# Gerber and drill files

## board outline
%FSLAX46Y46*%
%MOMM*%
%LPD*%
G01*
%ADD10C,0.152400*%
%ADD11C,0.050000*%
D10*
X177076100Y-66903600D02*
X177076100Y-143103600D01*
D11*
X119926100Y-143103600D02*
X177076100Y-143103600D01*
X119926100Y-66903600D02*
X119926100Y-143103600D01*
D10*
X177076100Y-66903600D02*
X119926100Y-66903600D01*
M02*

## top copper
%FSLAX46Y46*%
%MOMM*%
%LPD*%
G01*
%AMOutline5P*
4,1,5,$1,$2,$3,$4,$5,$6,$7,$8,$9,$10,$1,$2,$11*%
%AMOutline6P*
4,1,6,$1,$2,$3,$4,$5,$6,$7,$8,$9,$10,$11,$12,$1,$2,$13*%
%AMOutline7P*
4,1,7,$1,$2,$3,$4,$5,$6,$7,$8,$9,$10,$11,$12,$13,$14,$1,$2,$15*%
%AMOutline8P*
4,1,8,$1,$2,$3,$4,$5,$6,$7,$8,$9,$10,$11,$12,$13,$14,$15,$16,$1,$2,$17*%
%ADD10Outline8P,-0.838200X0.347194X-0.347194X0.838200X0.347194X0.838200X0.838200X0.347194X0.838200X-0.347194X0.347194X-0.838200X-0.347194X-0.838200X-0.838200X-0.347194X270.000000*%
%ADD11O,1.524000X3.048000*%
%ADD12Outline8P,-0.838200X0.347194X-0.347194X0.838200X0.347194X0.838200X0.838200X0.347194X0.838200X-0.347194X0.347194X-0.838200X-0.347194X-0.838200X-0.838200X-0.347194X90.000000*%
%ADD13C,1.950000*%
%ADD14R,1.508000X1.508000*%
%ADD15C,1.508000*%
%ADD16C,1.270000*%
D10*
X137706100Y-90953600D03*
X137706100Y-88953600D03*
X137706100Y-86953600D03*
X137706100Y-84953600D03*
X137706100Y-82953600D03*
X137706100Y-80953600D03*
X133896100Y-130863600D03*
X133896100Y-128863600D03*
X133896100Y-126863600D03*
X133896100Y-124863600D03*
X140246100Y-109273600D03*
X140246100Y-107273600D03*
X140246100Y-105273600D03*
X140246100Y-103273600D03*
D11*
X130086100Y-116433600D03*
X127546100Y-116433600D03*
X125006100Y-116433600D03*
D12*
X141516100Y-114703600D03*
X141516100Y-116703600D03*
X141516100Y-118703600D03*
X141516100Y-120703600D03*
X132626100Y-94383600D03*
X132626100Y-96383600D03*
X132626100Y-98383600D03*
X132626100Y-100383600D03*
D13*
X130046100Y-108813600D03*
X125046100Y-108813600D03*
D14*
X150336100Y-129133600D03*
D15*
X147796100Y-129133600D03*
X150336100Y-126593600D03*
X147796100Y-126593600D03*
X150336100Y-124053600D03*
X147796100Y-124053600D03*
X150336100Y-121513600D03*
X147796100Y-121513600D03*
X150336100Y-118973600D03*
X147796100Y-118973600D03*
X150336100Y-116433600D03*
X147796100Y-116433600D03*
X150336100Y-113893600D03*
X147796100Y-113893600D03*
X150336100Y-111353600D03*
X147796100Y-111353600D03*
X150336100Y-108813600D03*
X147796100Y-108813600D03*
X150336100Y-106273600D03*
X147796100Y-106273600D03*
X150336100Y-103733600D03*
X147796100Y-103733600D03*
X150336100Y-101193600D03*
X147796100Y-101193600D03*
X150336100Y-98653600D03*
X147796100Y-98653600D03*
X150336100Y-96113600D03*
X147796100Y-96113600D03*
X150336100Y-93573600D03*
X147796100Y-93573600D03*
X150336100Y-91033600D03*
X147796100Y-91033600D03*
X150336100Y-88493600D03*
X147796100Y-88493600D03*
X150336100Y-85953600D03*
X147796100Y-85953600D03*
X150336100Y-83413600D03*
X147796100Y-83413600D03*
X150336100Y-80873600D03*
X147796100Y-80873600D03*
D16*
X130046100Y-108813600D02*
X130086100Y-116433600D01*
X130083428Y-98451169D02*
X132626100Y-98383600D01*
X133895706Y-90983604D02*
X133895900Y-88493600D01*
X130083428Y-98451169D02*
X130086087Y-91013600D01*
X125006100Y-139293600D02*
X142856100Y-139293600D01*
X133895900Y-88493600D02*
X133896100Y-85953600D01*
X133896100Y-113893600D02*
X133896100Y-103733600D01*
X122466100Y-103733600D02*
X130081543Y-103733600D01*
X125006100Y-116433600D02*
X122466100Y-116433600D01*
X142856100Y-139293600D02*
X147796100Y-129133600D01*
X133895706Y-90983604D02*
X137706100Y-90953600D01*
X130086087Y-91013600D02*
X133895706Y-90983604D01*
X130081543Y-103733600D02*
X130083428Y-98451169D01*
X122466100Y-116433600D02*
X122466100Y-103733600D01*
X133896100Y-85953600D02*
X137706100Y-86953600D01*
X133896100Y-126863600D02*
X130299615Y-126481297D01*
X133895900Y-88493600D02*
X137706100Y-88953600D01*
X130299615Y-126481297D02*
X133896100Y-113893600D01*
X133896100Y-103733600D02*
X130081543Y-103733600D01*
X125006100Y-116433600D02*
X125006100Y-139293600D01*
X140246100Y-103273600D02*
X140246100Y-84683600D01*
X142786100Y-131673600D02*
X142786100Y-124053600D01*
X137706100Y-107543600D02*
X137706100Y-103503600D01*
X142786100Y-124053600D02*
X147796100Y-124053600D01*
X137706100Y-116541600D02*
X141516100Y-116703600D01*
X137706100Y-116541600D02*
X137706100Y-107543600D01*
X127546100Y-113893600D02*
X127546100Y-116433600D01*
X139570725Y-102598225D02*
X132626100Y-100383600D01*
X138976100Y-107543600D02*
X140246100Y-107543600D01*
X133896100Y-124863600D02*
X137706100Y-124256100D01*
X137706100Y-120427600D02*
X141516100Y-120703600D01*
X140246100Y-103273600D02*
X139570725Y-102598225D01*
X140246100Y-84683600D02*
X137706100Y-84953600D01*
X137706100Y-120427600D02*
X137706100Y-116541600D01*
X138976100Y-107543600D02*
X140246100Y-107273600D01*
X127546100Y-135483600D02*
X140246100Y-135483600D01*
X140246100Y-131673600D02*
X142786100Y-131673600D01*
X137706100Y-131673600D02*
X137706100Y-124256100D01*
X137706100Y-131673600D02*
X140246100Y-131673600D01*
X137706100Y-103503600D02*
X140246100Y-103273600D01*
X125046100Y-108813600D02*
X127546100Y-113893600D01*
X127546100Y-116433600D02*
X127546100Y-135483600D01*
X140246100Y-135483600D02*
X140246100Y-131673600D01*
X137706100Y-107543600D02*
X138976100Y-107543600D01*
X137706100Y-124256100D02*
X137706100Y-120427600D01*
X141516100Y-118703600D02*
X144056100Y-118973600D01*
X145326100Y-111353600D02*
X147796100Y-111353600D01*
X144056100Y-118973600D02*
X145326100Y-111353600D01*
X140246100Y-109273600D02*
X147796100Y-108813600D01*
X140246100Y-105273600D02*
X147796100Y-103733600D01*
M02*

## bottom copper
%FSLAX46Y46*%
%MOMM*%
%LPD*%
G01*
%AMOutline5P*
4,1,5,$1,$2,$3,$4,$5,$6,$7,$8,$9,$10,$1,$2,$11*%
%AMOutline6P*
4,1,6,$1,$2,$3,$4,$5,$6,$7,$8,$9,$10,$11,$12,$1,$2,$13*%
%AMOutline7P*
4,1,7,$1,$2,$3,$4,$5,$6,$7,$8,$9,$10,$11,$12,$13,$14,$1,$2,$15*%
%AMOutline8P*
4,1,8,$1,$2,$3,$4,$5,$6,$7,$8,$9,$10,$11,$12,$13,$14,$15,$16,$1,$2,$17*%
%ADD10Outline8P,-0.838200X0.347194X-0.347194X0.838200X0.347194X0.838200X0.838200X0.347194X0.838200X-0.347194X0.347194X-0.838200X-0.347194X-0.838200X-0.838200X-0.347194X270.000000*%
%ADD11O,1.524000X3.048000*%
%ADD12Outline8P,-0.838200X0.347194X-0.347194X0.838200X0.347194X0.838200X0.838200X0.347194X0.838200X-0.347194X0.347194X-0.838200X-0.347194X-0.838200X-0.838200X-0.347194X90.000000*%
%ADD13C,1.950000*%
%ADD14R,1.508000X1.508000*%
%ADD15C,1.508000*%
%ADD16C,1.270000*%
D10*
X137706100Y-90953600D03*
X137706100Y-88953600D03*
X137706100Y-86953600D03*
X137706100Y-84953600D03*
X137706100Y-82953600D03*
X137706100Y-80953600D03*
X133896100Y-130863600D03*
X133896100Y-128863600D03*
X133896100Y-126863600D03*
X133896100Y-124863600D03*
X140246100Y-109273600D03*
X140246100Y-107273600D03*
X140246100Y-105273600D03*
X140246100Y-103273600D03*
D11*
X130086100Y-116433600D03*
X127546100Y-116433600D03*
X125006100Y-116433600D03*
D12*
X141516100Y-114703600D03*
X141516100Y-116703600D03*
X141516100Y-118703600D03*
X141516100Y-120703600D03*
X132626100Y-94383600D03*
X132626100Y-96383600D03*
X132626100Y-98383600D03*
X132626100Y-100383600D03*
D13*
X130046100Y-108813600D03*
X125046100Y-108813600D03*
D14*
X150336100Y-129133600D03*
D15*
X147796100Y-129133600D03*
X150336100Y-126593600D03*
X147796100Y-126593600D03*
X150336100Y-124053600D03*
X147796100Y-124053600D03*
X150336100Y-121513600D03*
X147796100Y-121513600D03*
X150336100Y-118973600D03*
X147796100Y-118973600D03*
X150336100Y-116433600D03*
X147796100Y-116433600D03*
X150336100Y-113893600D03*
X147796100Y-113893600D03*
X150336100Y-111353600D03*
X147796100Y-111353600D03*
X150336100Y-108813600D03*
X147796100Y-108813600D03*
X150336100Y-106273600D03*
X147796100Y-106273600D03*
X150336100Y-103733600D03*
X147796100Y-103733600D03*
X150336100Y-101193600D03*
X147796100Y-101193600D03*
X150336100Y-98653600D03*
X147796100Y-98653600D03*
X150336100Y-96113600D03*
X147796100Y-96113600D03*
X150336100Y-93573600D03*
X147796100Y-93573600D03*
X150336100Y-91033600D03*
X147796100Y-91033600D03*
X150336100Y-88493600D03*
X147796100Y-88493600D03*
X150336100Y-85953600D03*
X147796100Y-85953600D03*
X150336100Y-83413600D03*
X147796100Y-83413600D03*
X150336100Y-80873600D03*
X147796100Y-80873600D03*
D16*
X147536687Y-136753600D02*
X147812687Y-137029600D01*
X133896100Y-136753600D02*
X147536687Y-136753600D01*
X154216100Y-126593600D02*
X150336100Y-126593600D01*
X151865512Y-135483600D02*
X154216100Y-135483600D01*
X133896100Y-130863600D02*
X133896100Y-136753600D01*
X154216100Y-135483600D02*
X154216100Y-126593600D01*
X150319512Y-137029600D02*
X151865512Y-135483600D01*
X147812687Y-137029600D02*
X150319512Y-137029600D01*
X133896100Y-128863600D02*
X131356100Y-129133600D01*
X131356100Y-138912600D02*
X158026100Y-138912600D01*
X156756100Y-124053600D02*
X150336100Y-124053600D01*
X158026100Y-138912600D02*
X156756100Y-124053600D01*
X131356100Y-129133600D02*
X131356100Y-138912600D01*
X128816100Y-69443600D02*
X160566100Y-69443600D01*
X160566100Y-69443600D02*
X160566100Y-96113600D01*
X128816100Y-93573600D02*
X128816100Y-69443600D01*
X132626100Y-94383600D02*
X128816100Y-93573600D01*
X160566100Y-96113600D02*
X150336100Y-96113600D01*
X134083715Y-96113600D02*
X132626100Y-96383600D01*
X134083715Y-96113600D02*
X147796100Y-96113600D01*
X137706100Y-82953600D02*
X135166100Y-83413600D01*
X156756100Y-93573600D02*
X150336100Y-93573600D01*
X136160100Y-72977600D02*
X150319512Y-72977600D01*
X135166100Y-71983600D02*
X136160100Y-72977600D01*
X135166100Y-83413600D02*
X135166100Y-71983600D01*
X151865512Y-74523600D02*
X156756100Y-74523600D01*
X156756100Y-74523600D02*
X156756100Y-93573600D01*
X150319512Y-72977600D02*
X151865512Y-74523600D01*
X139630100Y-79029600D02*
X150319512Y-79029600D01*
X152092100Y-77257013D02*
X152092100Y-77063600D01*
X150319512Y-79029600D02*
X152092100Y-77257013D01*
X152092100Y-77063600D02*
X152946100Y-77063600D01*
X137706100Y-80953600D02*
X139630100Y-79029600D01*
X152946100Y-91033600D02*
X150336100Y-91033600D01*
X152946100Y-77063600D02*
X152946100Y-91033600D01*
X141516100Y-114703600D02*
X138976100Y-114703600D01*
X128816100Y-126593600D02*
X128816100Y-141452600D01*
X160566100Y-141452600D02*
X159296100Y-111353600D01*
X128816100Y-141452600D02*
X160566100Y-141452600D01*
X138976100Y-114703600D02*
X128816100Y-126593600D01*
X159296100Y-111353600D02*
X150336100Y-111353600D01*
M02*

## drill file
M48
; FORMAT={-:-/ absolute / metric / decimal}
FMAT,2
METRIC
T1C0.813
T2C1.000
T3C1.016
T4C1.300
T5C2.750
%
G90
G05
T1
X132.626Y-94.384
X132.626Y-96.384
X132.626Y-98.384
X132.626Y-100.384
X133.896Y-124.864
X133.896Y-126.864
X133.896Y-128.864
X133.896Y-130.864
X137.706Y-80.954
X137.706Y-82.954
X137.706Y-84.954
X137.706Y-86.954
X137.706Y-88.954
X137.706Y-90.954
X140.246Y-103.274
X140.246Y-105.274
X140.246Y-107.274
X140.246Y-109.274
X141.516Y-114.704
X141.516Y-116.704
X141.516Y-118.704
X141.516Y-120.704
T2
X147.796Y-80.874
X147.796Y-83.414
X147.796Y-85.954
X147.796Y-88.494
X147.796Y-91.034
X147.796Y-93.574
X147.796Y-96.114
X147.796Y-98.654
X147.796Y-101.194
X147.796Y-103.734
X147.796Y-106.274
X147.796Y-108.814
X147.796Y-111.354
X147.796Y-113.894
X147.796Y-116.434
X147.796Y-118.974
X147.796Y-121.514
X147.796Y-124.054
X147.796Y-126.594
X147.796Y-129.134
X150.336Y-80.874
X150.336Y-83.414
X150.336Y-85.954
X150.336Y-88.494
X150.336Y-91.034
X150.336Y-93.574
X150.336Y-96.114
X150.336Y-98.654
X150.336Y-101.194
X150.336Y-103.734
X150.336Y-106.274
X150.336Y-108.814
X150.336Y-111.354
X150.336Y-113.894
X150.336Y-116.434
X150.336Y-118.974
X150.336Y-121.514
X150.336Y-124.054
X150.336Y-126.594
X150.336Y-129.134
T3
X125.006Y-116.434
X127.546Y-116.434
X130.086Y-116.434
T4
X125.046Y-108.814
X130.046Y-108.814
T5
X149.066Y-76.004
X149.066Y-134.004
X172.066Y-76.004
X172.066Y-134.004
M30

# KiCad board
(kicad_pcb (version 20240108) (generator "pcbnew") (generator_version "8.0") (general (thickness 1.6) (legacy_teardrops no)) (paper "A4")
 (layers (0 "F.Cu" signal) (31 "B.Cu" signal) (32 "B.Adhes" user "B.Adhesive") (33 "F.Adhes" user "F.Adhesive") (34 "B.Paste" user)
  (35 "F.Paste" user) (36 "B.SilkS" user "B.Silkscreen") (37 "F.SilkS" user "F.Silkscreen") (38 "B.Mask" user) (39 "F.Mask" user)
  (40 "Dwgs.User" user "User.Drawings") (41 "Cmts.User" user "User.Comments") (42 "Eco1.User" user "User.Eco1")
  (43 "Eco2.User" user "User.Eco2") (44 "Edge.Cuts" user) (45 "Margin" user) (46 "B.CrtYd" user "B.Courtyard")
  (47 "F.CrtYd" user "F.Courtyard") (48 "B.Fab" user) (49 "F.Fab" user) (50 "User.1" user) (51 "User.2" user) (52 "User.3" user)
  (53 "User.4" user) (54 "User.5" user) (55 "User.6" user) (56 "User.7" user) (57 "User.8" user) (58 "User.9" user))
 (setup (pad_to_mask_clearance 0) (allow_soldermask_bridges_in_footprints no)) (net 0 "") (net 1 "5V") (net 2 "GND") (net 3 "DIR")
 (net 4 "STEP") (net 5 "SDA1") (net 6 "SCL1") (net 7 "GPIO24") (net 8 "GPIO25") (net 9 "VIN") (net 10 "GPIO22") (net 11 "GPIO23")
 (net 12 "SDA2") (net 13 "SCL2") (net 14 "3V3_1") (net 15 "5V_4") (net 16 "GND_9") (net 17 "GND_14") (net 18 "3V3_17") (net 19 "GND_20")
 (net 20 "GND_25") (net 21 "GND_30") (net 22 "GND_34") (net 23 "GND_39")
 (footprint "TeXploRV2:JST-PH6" (layer "F.Cu") (at 137.7061 85.9536 -90)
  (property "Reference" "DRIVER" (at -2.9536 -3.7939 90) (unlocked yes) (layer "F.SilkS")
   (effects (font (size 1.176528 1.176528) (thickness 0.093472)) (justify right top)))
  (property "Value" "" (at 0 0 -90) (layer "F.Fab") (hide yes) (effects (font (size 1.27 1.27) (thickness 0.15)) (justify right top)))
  (pad "1" thru_hole roundrect (at 5 0 270) (size 1.6764 1.6764) (drill 0.8128) (layers "*.Cu" "*.Mask") (remove_unused_layers no)
   (roundrect_rratio 0.25) (chamfer_ratio 0.2928932188) (chamfer top_left top_right bottom_left bottom_right) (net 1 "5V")
   (solder_mask_margin 0.1016) (thermal_bridge_angle 0))
  (pad "2" thru_hole roundrect (at 3 0 270) (size 1.6764 1.6764) (drill 0.8128) (layers "*.Cu" "*.Mask") (remove_unused_layers no)
   (roundrect_rratio 0.25) (chamfer_ratio 0.2928932188) (chamfer top_left top_right bottom_left bottom_right) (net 1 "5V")
   (solder_mask_margin 0.1016) (thermal_bridge_angle 0))
  (pad "3" thru_hole roundrect (at 1 0 270) (size 1.6764 1.6764) (drill 0.8128) (layers "*.Cu" "*.Mask") (remove_unused_layers no)
   (roundrect_rratio 0.25) (chamfer_ratio 0.2928932188) (chamfer top_left top_right bottom_left bottom_right) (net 1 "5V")
   (solder_mask_margin 0.1016) (thermal_bridge_angle 0))
  (pad "4" thru_hole roundrect (at -1 0 270) (size 1.6764 1.6764) (drill 0.8128) (layers "*.Cu" "*.Mask") (remove_unused_layers no)
   (roundrect_rratio 0.25) (chamfer_ratio 0.2928932188) (chamfer top_left top_right bottom_left bottom_right) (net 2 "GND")
   (solder_mask_margin 0.1016) (thermal_bridge_angle 0))
  (pad "5" thru_hole roundrect (at -3 0 270) (size 1.6764 1.6764) (drill 0.8128) (layers "*.Cu" "*.Mask") (remove_unused_layers no)
   (roundrect_rratio 0.25) (chamfer_ratio 0.2928932188) (chamfer top_left top_right bottom_left bottom_right) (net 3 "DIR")
   (solder_mask_margin 0.1016) (thermal_bridge_angle 0))
  (pad "6" thru_hole roundrect (at -5 0 270) (size 1.6764 1.6764) (drill 0.8128) (layers "*.Cu" "*.Mask") (remove_unused_layers no)
   (roundrect_rratio 0.25) (chamfer_ratio 0.2928932188) (chamfer top_left top_right bottom_left bottom_right) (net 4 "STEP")
   (solder_mask_margin 0.1016) (thermal_bridge_angle 0)))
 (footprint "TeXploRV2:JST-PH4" (layer "F.Cu") (at 133.8961 127.8636 -90)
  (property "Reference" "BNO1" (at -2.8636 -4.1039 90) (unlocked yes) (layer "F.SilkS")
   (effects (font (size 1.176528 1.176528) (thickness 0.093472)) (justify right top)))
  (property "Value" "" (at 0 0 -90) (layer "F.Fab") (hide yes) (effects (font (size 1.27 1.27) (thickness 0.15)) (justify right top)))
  (pad "1" thru_hole roundrect (at 3 0 270) (size 1.6764 1.6764) (drill 0.8128) (layers "*.Cu" "*.Mask") (remove_unused_layers no)
   (roundrect_rratio 0.25) (chamfer_ratio 0.2928932188) (chamfer top_left top_right bottom_left bottom_right) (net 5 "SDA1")
   (solder_mask_margin 0.1016) (thermal_bridge_angle 0))
  (pad "2" thru_hole roundrect (at 1 0 270) (size 1.6764 1.6764) (drill 0.8128) (layers "*.Cu" "*.Mask") (remove_unused_layers no)
   (roundrect_rratio 0.25) (chamfer_ratio 0.2928932188) (chamfer top_left top_right bottom_left bottom_right) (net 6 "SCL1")
   (solder_mask_margin 0.1016) (thermal_bridge_angle 0))
  (pad "3" thru_hole roundrect (at -1 0 270) (size 1.6764 1.6764) (drill 0.8128) (layers "*.Cu" "*.Mask") (remove_unused_layers no)
   (roundrect_rratio 0.25) (chamfer_ratio 0.2928932188) (chamfer top_left top_right bottom_left bottom_right) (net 1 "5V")
   (solder_mask_margin 0.1016) (thermal_bridge_angle 0))
  (pad "4" thru_hole roundrect (at -3 0 270) (size 1.6764 1.6764) (drill 0.8128) (layers "*.Cu" "*.Mask") (remove_unused_layers no)
   (roundrect_rratio 0.25) (chamfer_ratio 0.2928932188) (chamfer top_left top_right bottom_left bottom_right) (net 2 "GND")
   (solder_mask_margin 0.1016) (thermal_bridge_angle 0)))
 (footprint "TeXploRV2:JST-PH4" (layer "F.Cu") (at 140.2461 106.2736 -90)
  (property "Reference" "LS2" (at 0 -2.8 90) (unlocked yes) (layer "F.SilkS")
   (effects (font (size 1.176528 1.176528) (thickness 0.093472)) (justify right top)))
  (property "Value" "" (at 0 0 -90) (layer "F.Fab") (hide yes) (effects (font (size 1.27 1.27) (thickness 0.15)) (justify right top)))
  (pad "1" thru_hole roundrect (at 3 0 270) (size 1.6764 1.6764) (drill 0.8128) (layers "*.Cu" "*.Mask") (remove_unused_layers no)
   (roundrect_rratio 0.25) (chamfer_ratio 0.2928932188) (chamfer top_left top_right bottom_left bottom_right) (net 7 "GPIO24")
   (solder_mask_margin 0.1016) (thermal_bridge_angle 0))
  (pad "2" thru_hole roundrect (at 1 0 270) (size 1.6764 1.6764) (drill 0.8128) (layers "*.Cu" "*.Mask") (remove_unused_layers no)
   (roundrect_rratio 0.25) (chamfer_ratio 0.2928932188) (chamfer top_left top_right bottom_left bottom_right) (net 2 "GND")
   (solder_mask_margin 0.1016) (thermal_bridge_angle 0))
  (pad "3" thru_hole roundrect (at -1 0 270) (size 1.6764 1.6764) (drill 0.8128) (layers "*.Cu" "*.Mask") (remove_unused_layers no)
   (roundrect_rratio 0.25) (chamfer_ratio 0.2928932188) (chamfer top_left top_right bottom_left bottom_right) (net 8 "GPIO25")
   (solder_mask_margin 0.1016) (thermal_bridge_angle 0))
  (pad "4" thru_hole roundrect (at -3 0 270) (size 1.6764 1.6764) (drill 0.8128) (layers "*.Cu" "*.Mask") (remove_unused_layers no)
   (roundrect_rratio 0.25) (chamfer_ratio 0.2928932188) (chamfer top_left top_right bottom_left bottom_right) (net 2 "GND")
   (solder_mask_margin 0.1016) (thermal_bridge_angle 0)))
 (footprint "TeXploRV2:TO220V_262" (layer "F.Cu") (at 127.5461 118.9736 180)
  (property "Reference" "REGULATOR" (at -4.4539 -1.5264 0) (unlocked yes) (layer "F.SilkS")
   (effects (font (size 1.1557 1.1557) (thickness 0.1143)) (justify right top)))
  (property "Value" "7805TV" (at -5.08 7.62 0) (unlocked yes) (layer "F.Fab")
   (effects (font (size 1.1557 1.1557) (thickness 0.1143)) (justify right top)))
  (pad "1" thru_hole oval (at -2.54 2.54 270) (size 3.048 1.524) (drill 1.016) (layers "*.Cu" "*.Mask") (remove_unused_layers no)
   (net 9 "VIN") (solder_mask_margin 0.1016) (thermal_bridge_angle 0))
  (pad "2" thru_hole oval (at 0 2.54 270) (size 3.048 1.524) (drill 1.016) (layers "*.Cu" "*.Mask") (remove_unused_layers no) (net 2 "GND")
   (solder_mask_margin 0.1016) (thermal_bridge_angle 0))
  (pad "3" thru_hole oval (at 2.54 2.54 270) (size 3.048 1.524) (drill 1.016) (layers "*.Cu" "*.Mask") (remove_unused_layers no)
   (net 1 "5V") (solder_mask_margin 0.1016) (thermal_bridge_angle 0)))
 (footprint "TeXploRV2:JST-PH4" (layer "F.Cu") (at 141.5161 117.7036 90)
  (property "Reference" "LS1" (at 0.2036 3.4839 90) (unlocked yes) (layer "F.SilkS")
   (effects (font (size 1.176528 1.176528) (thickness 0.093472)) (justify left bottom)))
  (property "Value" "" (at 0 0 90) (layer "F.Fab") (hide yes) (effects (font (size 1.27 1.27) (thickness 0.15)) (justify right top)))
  (pad "1" thru_hole roundrect (at 3 0 90) (size 1.6764 1.6764) (drill 0.8128) (layers "*.Cu" "*.Mask") (remove_unused_layers no)
   (roundrect_rratio 0.25) (chamfer_ratio 0.2928932188) (chamfer top_left top_right bottom_left bottom_right) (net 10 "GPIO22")
   (solder_mask_margin 0.1016) (thermal_bridge_angle 0))
  (pad "2" thru_hole roundrect (at 1 0 90) (size 1.6764 1.6764) (drill 0.8128) (layers "*.Cu" "*.Mask") (remove_unused_layers no)
   (roundrect_rratio 0.25) (chamfer_ratio 0.2928932188) (chamfer top_left top_right bottom_left bottom_right) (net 2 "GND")
   (solder_mask_margin 0.1016) (thermal_bridge_angle 0))
  (pad "3" thru_hole roundrect (at -1 0 90) (size 1.6764 1.6764) (drill 0.8128) (layers "*.Cu" "*.Mask") (remove_unused_layers no)
   (roundrect_rratio 0.25) (chamfer_ratio 0.2928932188) (chamfer top_left top_right bottom_left bottom_right) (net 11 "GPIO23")
   (solder_mask_margin 0.1016) (thermal_bridge_angle 0))
  (pad "4" thru_hole roundrect (at -3 0 90) (size 1.6764 1.6764) (drill 0.8128) (layers "*.Cu" "*.Mask") (remove_unused_layers no)
   (roundrect_rratio 0.25) (chamfer_ratio 0.2928932188) (chamfer top_left top_right bottom_left bottom_right) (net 2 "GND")
   (solder_mask_margin 0.1016) (thermal_bridge_angle 0)))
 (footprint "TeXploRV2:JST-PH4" (layer "F.Cu") (at 132.6261 97.3836 90)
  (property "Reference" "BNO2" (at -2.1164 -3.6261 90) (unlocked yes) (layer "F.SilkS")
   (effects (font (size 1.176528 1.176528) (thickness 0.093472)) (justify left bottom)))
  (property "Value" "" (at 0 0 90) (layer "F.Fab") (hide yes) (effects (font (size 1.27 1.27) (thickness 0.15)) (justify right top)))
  (pad "1" thru_hole roundrect (at 3 0 90) (size 1.6764 1.6764) (drill 0.8128) (layers "*.Cu" "*.Mask") (remove_unused_layers no)
   (roundrect_rratio 0.25) (chamfer_ratio 0.2928932188) (chamfer top_left top_right bottom_left bottom_right) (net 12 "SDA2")
   (solder_mask_margin 0.1016) (thermal_bridge_angle 0))
  (pad "2" thru_hole roundrect (at 1 0 90) (size 1.6764 1.6764) (drill 0.8128) (layers "*.Cu" "*.Mask") (remove_unused_layers no)
   (roundrect_rratio 0.25) (chamfer_ratio 0.2928932188) (chamfer top_left top_right bottom_left bottom_right) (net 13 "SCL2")
   (solder_mask_margin 0.1016) (thermal_bridge_angle 0))
  (pad "3" thru_hole roundrect (at -1 0 90) (size 1.6764 1.6764) (drill 0.8128) (layers "*.Cu" "*.Mask") (remove_unused_layers no)
   (roundrect_rratio 0.25) (chamfer_ratio 0.2928932188) (chamfer top_left top_right bottom_left bottom_right) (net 1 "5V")
   (solder_mask_margin 0.1016) (thermal_bridge_angle 0))
  (pad "4" thru_hole roundrect (at -3 0 90) (size 1.6764 1.6764) (drill 0.8128) (layers "*.Cu" "*.Mask") (remove_unused_layers no)
   (roundrect_rratio 0.25) (chamfer_ratio 0.2928932188) (chamfer top_left top_right bottom_left bottom_right) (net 2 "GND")
   (solder_mask_margin 0.1016) (thermal_bridge_angle 0)))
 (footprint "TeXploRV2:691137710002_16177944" (layer "F.Cu") (at 127.5461 108.8136 180)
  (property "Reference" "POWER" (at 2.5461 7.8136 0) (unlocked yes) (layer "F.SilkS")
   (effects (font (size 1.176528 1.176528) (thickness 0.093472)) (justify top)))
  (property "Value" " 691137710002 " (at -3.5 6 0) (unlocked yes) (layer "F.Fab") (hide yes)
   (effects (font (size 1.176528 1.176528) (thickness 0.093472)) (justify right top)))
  (pad "1" thru_hole circle (at -2.5 0 180) (size 1.95 1.95) (drill 1.3) (layers "*.Cu" "*.Mask") (remove_unused_layers no) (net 9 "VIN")
   (solder_mask_margin 0.1016) (thermal_bridge_angle 0))
  (pad "2" thru_hole circle (at 2.5 0 180) (size 1.95 1.95) (drill 1.3) (layers "*.Cu" "*.Mask") (remove_unused_layers no) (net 2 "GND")
   (solder_mask_margin 0.1016) (thermal_bridge_angle 0)))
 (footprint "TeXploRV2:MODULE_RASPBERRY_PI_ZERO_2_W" (layer "F.Cu") (at 160.5661 105.0036 90)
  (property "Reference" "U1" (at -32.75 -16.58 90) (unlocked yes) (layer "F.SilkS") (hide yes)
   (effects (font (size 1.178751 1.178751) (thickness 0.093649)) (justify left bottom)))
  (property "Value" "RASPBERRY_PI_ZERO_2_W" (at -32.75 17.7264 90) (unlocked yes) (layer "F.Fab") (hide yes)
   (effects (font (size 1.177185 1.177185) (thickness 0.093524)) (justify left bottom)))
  (pad "" np_thru_hole circle (at -29 -11.5 90) (size 2.75 2.75) (drill 2.75) (layers "*.Cu" "*.Mask"))
  (pad "" np_thru_hole circle (at -29 11.5 90) (size 2.75 2.75) (drill 2.75) (layers "*.Cu" "*.Mask"))
  (pad "" np_thru_hole circle (at 29 -11.5 90) (size 2.75 2.75) (drill 2.75) (layers "*.Cu" "*.Mask"))
  (pad "" np_thru_hole circle (at 29 11.5 90) (size 2.75 2.75) (drill 2.75) (layers "*.Cu" "*.Mask"))
  (pad "1" thru_hole rect (at -24.13 -10.23 90) (size 1.508 1.508) (drill 1) (layers "*.Cu" "*.Mask") (remove_unused_layers no)
   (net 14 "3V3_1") (solder_mask_margin 0.1016) (thermal_bridge_angle 0))
  (pad "2" thru_hole circle (at -24.13 -12.77 90) (size 1.508 1.508) (drill 1) (layers "*.Cu" "*.Mask") (remove_unused_layers no)
   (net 1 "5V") (solder_mask_margin 0.1016) (thermal_bridge_angle 0))
  (pad "3" thru_hole circle (at -21.59 -10.23 90) (size 1.508 1.508) (drill 1) (layers "*.Cu" "*.Mask") (remove_unused_layers no)
   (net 5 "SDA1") (solder_mask_margin 0.1016) (thermal_bridge_angle 0))
  (pad "4" thru_hole circle (at -21.59 -12.77 90) (size 1.508 1.508) (drill 1) (layers "*.Cu" "*.Mask") (remove_unused_layers no)
   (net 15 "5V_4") (solder_mask_margin 0.1016) (thermal_bridge_angle 0))
  (pad "5" thru_hole circle (at -19.05 -10.23 90) (size 1.508 1.508) (drill 1) (layers "*.Cu" "*.Mask") (remove_unused_layers no)
   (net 6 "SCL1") (solder_mask_margin 0.1016) (thermal_bridge_angle 0))
  (pad "6" thru_hole circle (at -19.05 -12.77 90) (size 1.508 1.508) (drill 1) (layers "*.Cu" "*.Mask") (remove_unused_layers no)
   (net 2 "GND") (solder_mask_margin 0.1016) (thermal_bridge_angle 0))
  (pad "7" thru_hole circle (at -16.51 -10.23 90) (size 1.508 1.508) (drill 1) (layers "*.Cu" "*.Mask") (remove_unused_layers no)
   (solder_mask_margin 0.1016) (thermal_bridge_angle 0))
  (pad "8" thru_hole circle (at -16.51 -12.77 90) (size 1.508 1.508) (drill 1) (layers "*.Cu" "*.Mask") (remove_unused_layers no)
   (solder_mask_margin 0.1016) (thermal_bridge_angle 0))
  (pad "9" thru_hole circle (at -13.97 -10.23 90) (size 1.508 1.508) (drill 1) (layers "*.Cu" "*.Mask") (remove_unused_layers no)
   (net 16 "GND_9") (solder_mask_margin 0.1016) (thermal_bridge_angle 0))
  (pad "10" thru_hole circle (at -13.97 -12.77 90) (size 1.508 1.508) (drill 1) (layers "*.Cu" "*.Mask") (remove_unused_layers no)
   (solder_mask_margin 0.1016) (thermal_bridge_angle 0))
  (pad "11" thru_hole circle (at -11.43 -10.23 90) (size 1.508 1.508) (drill 1) (layers "*.Cu" "*.Mask") (remove_unused_layers no)
   (solder_mask_margin 0.1016) (thermal_bridge_angle 0))
  (pad "12" thru_hole circle (at -11.43 -12.77 90) (size 1.508 1.508) (drill 1) (layers "*.Cu" "*.Mask") (remove_unused_layers no)
   (solder_mask_margin 0.1016) (thermal_bridge_angle 0))
  (pad "13" thru_hole circle (at -8.89 -10.23 90) (size 1.508 1.508) (drill 1) (layers "*.Cu" "*.Mask") (remove_unused_layers no)
   (solder_mask_margin 0.1016) (thermal_bridge_angle 0))
  (pad "14" thru_hole circle (at -8.89 -12.77 90) (size 1.508 1.508) (drill 1) (layers "*.Cu" "*.Mask") (remove_unused_layers no)
   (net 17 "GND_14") (solder_mask_margin 0.1016) (thermal_bridge_angle 0))
  (pad "15" thru_hole circle (at -6.35 -10.23 90) (size 1.508 1.508) (drill 1) (layers "*.Cu" "*.Mask") (remove_unused_layers no)
   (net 10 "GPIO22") (solder_mask_margin 0.1016) (thermal_bridge_angle 0))
  (pad "16" thru_hole circle (at -6.35 -12.77 90) (size 1.508 1.508) (drill 1) (layers "*.Cu" "*.Mask") (remove_unused_layers no)
   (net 11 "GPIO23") (solder_mask_margin 0.1016) (thermal_bridge_angle 0))
  (pad "17" thru_hole circle (at -3.81 -10.23 90) (size 1.508 1.508) (drill 1) (layers "*.Cu" "*.Mask") (remove_unused_layers no)
   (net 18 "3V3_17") (solder_mask_margin 0.1016) (thermal_bridge_angle 0))
  (pad "18" thru_hole circle (at -3.81 -12.77 90) (size 1.508 1.508) (drill 1) (layers "*.Cu" "*.Mask") (remove_unused_layers no)
   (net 7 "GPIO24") (solder_mask_margin 0.1016) (thermal_bridge_angle 0))
  (pad "19" thru_hole circle (at -1.27 -10.23 90) (size 1.508 1.508) (drill 1) (layers "*.Cu" "*.Mask") (remove_unused_layers no)
   (solder_mask_margin 0.1016) (thermal_bridge_angle 0))
  (pad "20" thru_hole circle (at -1.27 -12.77 90) (size 1.508 1.508) (drill 1) (layers "*.Cu" "*.Mask") (remove_unused_layers no)
   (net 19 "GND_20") (solder_mask_margin 0.1016) (thermal_bridge_angle 0))
  (pad "21" thru_hole circle (at 1.27 -10.23 90) (size 1.508 1.508) (drill 1) (layers "*.Cu" "*.Mask") (remove_unused_layers no)
   (solder_mask_margin 0.1016) (thermal_bridge_angle 0))
  (pad "22" thru_hole circle (at 1.27 -12.77 90) (size 1.508 1.508) (drill 1) (layers "*.Cu" "*.Mask") (remove_unused_layers no)
   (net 8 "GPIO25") (solder_mask_margin 0.1016) (thermal_bridge_angle 0))
  (pad "23" thru_hole circle (at 3.81 -10.23 90) (size 1.508 1.508) (drill 1) (layers "*.Cu" "*.Mask") (remove_unused_layers no)
   (solder_mask_margin 0.1016) (thermal_bridge_angle 0))
  (pad "24" thru_hole circle (at 3.81 -12.77 90) (size 1.508 1.508) (drill 1) (layers "*.Cu" "*.Mask") (remove_unused_layers no)
   (solder_mask_margin 0.1016) (thermal_bridge_angle 0))
  (pad "25" thru_hole circle (at 6.35 -10.23 90) (size 1.508 1.508) (drill 1) (layers "*.Cu" "*.Mask") (remove_unused_layers no)
   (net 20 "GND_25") (solder_mask_margin 0.1016) (thermal_bridge_angle 0))
  (pad "26" thru_hole circle (at 6.35 -12.77 90) (size 1.508 1.508) (drill 1) (layers "*.Cu" "*.Mask") (remove_unused_layers no)
   (solder_mask_margin 0.1016) (thermal_bridge_angle 0))
  (pad "27" thru_hole circle (at 8.89 -10.23 90) (size 1.508 1.508) (drill 1) (layers "*.Cu" "*.Mask") (remove_unused_layers no)
   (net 12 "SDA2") (solder_mask_margin 0.1016) (thermal_bridge_angle 0))
  (pad "28" thru_hole circle (at 8.89 -12.77 90) (size 1.508 1.508) (drill 1) (layers "*.Cu" "*.Mask") (remove_unused_layers no)
   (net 13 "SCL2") (solder_mask_margin 0.1016) (thermal_bridge_angle 0))
  (pad "29" thru_hole circle (at 11.43 -10.23 90) (size 1.508 1.508) (drill 1) (layers "*.Cu" "*.Mask") (remove_unused_layers no)
   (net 3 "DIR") (solder_mask_margin 0.1016) (thermal_bridge_angle 0))
  (pad "30" thru_hole circle (at 11.43 -12.77 90) (size 1.508 1.508) (drill 1) (layers "*.Cu" "*.Mask") (remove_unused_layers no)
   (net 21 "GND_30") (solder_mask_margin 0.1016) (thermal_bridge_angle 0))
  (pad "31" thru_hole circle (at 13.97 -10.23 90) (size 1.508 1.508) (drill 1) (layers "*.Cu" "*.Mask") (remove_unused_layers no)
   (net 4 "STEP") (solder_mask_margin 0.1016) (thermal_bridge_angle 0))
  (pad "32" thru_hole circle (at 13.97 -12.77 90) (size 1.508 1.508) (drill 1) (layers "*.Cu" "*.Mask") (remove_unused_layers no)
   (solder_mask_margin 0.1016) (thermal_bridge_angle 0))
  (pad "33" thru_hole circle (at 16.51 -10.23 90) (size 1.508 1.508) (drill 1) (layers "*.Cu" "*.Mask") (remove_unused_layers no)
   (solder_mask_margin 0.1016) (thermal_bridge_angle 0))
  (pad "34" thru_hole circle (at 16.51 -12.77 90) (size 1.508 1.508) (drill 1) (layers "*.Cu" "*.Mask") (remove_unused_layers no)
   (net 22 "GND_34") (solder_mask_margin 0.1016) (thermal_bridge_angle 0))
  (pad "35" thru_hole circle (at 19.05 -10.23 90) (size 1.508 1.508) (drill 1) (layers "*.Cu" "*.Mask") (remove_unused_layers no)
   (solder_mask_margin 0.1016) (thermal_bridge_angle 0))
  (pad "36" thru_hole circle (at 19.05 -12.77 90) (size 1.508 1.508) (drill 1) (layers "*.Cu" "*.Mask") (remove_unused_layers no)
   (solder_mask_margin 0.1016) (thermal_bridge_angle 0))
  (pad "37" thru_hole circle (at 21.59 -10.23 90) (size 1.508 1.508) (drill 1) (layers "*.Cu" "*.Mask") (remove_unused_layers no)
   (solder_mask_margin 0.1016) (thermal_bridge_angle 0))
  (pad "38" thru_hole circle (at 21.59 -12.77 90) (size 1.508 1.508) (drill 1) (layers "*.Cu" "*.Mask") (remove_unused_layers no)
   (solder_mask_margin 0.1016) (thermal_bridge_angle 0))
  (pad "39" thru_hole circle (at 24.13 -10.23 90) (size 1.508 1.508) (drill 1) (layers "*.Cu" "*.Mask") (remove_unused_layers no)
   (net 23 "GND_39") (solder_mask_margin 0.1016) (thermal_bridge_angle 0))
  (pad "40" thru_hole circle (at 24.13 -12.77 90) (size 1.508 1.508) (drill 1) (layers "*.Cu" "*.Mask") (remove_unused_layers no)
   (solder_mask_margin 0.1016) (thermal_bridge_angle 0)))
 (gr_line (start 177.0761 66.9036) (end 177.0761 143.1036) (stroke (width 0.1524) (type solid)) (layer "Edge.Cuts"))
 (gr_line (start 119.9261 143.1036) (end 177.0761 143.1036) (stroke (width 0.05) (type solid)) (layer "Edge.Cuts"))
 (gr_line (start 119.9261 66.9036) (end 119.9261 143.1036) (stroke (width 0.05) (type solid)) (layer "Edge.Cuts"))
 (gr_line (start 177.0761 66.9036) (end 119.9261 66.9036) (stroke (width 0.1524) (type solid)) (layer "Edge.Cuts"))
 (segment (start 130.0461 108.8136) (end 130.0861 116.4336) (width 1.27) (layer "F.Cu") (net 9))
 (segment (start 130.083428 98.451169) (end 132.6261 98.3836) (width 1.27) (layer "F.Cu") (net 1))
 (segment (start 133.895706 90.983604) (end 133.8959 88.4936) (width 1.27) (layer "F.Cu") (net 1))
 (segment (start 130.083428 98.451169) (end 130.086087 91.0136) (width 1.27) (layer "F.Cu") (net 1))
 (segment (start 125.0061 139.2936) (end 142.8561 139.2936) (width 1.27) (layer "F.Cu") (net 1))
 (segment (start 133.8959 88.4936) (end 133.8961 85.9536) (width 1.27) (layer "F.Cu") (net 1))
 (segment (start 133.8961 113.8936) (end 133.8961 103.7336) (width 1.27) (layer "F.Cu") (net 1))
 (segment (start 122.4661 103.7336) (end 130.081543 103.7336) (width 1.27) (layer "F.Cu") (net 1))
 (segment (start 125.0061 116.4336) (end 122.4661 116.4336) (width 1.27) (layer "F.Cu") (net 1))
 (segment (start 142.8561 139.2936) (end 147.7961 129.1336) (width 1.27) (layer "F.Cu") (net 1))
 (segment (start 133.895706 90.983604) (end 137.7061 90.9536) (width 1.27) (layer "F.Cu") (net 1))
 (segment (start 130.086087 91.0136) (end 133.895706 90.983604) (width 1.27) (layer "F.Cu") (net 1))
 (segment (start 130.081543 103.7336) (end 130.083428 98.451169) (width 1.27) (layer "F.Cu") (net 1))
 (segment (start 122.4661 116.4336) (end 122.4661 103.7336) (width 1.27) (layer "F.Cu") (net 1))
 (segment (start 133.8961 85.9536) (end 137.7061 86.9536) (width 1.27) (layer "F.Cu") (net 1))
 (segment (start 133.8961 126.8636) (end 130.299615 126.481297) (width 1.27) (layer "F.Cu") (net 1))
 (segment (start 133.8959 88.4936) (end 137.7061 88.9536) (width 1.27) (layer "F.Cu") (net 1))
 (segment (start 130.299615 126.481297) (end 133.8961 113.8936) (width 1.27) (layer "F.Cu") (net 1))
 (segment (start 133.8961 103.7336) (end 130.081543 103.7336) (width 1.27) (layer "F.Cu") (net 1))
 (segment (start 125.0061 116.4336) (end 125.0061 139.2936) (width 1.27) (layer "F.Cu") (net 1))
 (segment (start 140.2461 103.2736) (end 140.2461 84.6836) (width 1.27) (layer "F.Cu") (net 2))
 (segment (start 142.7861 131.6736) (end 142.7861 124.0536) (width 1.27) (layer "F.Cu") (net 2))
 (segment (start 137.7061 107.5436) (end 137.7061 103.5036) (width 1.27) (layer "F.Cu") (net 2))
 (segment (start 142.7861 124.0536) (end 147.7961 124.0536) (width 1.27) (layer "F.Cu") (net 2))
 (segment (start 137.7061 116.5416) (end 141.5161 116.7036) (width 1.27) (layer "F.Cu") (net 2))
 (segment (start 137.7061 116.5416) (end 137.7061 107.5436) (width 1.27) (layer "F.Cu") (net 2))
 (segment (start 127.5461 113.8936) (end 127.5461 116.4336) (width 1.27) (layer "F.Cu") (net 2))
 (segment (start 139.570725 102.598225) (end 132.6261 100.3836) (width 1.27) (layer "F.Cu") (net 2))
 (segment (start 138.9761 107.5436) (end 140.2461 107.5436) (width 1.27) (layer "F.Cu") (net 2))
 (segment (start 133.8961 124.8636) (end 137.7061 124.2561) (width 1.27) (layer "F.Cu") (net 2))
 (segment (start 137.7061 120.4276) (end 141.5161 120.7036) (width 1.27) (layer "F.Cu") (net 2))
 (segment (start 140.2461 103.2736) (end 139.570725 102.598225) (width 1.27) (layer "F.Cu") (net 2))
 (segment (start 140.2461 84.6836) (end 137.7061 84.9536) (width 1.27) (layer "F.Cu") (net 2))
 (segment (start 137.7061 120.4276) (end 137.7061 116.5416) (width 1.27) (layer "F.Cu") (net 2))
 (segment (start 138.9761 107.5436) (end 140.2461 107.2736) (width 1.27) (layer "F.Cu") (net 2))
 (segment (start 127.5461 135.4836) (end 140.2461 135.4836) (width 1.27) (layer "F.Cu") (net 2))
 (segment (start 140.2461 131.6736) (end 142.7861 131.6736) (width 1.27) (layer "F.Cu") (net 2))
 (segment (start 137.7061 131.6736) (end 137.7061 124.2561) (width 1.27) (layer "F.Cu") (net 2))
 (segment (start 137.7061 131.6736) (end 140.2461 131.6736) (width 1.27) (layer "F.Cu") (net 2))
 (segment (start 137.7061 103.5036) (end 140.2461 103.2736) (width 1.27) (layer "F.Cu") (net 2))
 (segment (start 125.0461 108.8136) (end 127.5461 113.8936) (width 1.27) (layer "F.Cu") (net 2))
 (segment (start 127.5461 116.4336) (end 127.5461 135.4836) (width 1.27) (layer "F.Cu") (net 2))
 (segment (start 140.2461 135.4836) (end 140.2461 131.6736) (width 1.27) (layer "F.Cu") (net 2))
 (segment (start 137.7061 107.5436) (end 138.9761 107.5436) (width 1.27) (layer "F.Cu") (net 2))
 (segment (start 137.7061 124.2561) (end 137.7061 120.4276) (width 1.27) (layer "F.Cu") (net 2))
 (segment (start 147.536687 136.7536) (end 147.812687 137.0296) (width 1.27) (layer "B.Cu") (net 5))
 (segment (start 133.8961 136.7536) (end 147.536687 136.7536) (width 1.27) (layer "B.Cu") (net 5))
 (segment (start 154.2161 126.5936) (end 150.3361 126.5936) (width 1.27) (layer "B.Cu") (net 5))
 (segment (start 151.865512 135.4836) (end 154.2161 135.4836) (width 1.27) (layer "B.Cu") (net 5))
 (segment (start 133.8961 130.8636) (end 133.8961 136.7536) (width 1.27) (layer "B.Cu") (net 5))
 (segment (start 154.2161 135.4836) (end 154.2161 126.5936) (width 1.27) (layer "B.Cu") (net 5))
 (segment (start 150.319512 137.0296) (end 151.865512 135.4836) (width 1.27) (layer "B.Cu") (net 5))
 (segment (start 147.812687 137.0296) (end 150.319512 137.0296) (width 1.27) (layer "B.Cu") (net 5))
 (segment (start 133.8961 128.8636) (end 131.3561 129.1336) (width 1.27) (layer "B.Cu") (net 6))
 (segment (start 131.3561 138.9126) (end 158.0261 138.9126) (width 1.27) (layer "B.Cu") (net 6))
 (segment (start 156.7561 124.0536) (end 150.3361 124.0536) (width 1.27) (layer "B.Cu") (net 6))
 (segment (start 158.0261 138.9126) (end 156.7561 124.0536) (width 1.27) (layer "B.Cu") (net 6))
 (segment (start 131.3561 129.1336) (end 131.3561 138.9126) (width 1.27) (layer "B.Cu") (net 6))
 (segment (start 128.8161 69.4436) (end 160.5661 69.4436) (width 1.27) (layer "B.Cu") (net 12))
 (segment (start 160.5661 69.4436) (end 160.5661 96.1136) (width 1.27) (layer "B.Cu") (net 12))
 (segment (start 128.8161 93.5736) (end 128.8161 69.4436) (width 1.27) (layer "B.Cu") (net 12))
 (segment (start 132.6261 94.3836) (end 128.8161 93.5736) (width 1.27) (layer "B.Cu") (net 12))
 (segment (start 160.5661 96.1136) (end 150.3361 96.1136) (width 1.27) (layer "B.Cu") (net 12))
 (segment (start 134.083715 96.1136) (end 132.6261 96.3836) (width 1.27) (layer "B.Cu") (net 13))
 (segment (start 134.083715 96.1136) (end 147.7961 96.1136) (width 1.27) (layer "B.Cu") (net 13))
 (segment (start 137.7061 82.9536) (end 135.1661 83.4136) (width 1.27) (layer "B.Cu") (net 3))
 (segment (start 156.7561 93.5736) (end 150.3361 93.5736) (width 1.27) (layer "B.Cu") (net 3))
 (segment (start 136.1601 72.9776) (end 150.319512 72.9776) (width 1.27) (layer "B.Cu") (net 3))
 (segment (start 135.1661 71.9836) (end 136.1601 72.9776) (width 1.27) (layer "B.Cu") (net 3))
 (segment (start 135.1661 83.4136) (end 135.1661 71.9836) (width 1.27) (layer "B.Cu") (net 3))
 (segment (start 151.865512 74.5236) (end 156.7561 74.5236) (width 1.27) (layer "B.Cu") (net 3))
 (segment (start 156.7561 74.5236) (end 156.7561 93.5736) (width 1.27) (layer "B.Cu") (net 3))
 (segment (start 150.319512 72.9776) (end 151.865512 74.5236) (width 1.27) (layer "B.Cu") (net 3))
 (segment (start 139.6301 79.0296) (end 150.319512 79.0296) (width 1.27) (layer "B.Cu") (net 4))
 (segment (start 152.0921 77.257013) (end 152.0921 77.0636) (width 1.27) (layer "B.Cu") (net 4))
 (segment (start 150.319512 79.0296) (end 152.0921 77.257013) (width 1.27) (layer "B.Cu") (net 4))
 (segment (start 152.0921 77.0636) (end 152.9461 77.0636) (width 1.27) (layer "B.Cu") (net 4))
 (segment (start 137.7061 80.9536) (end 139.6301 79.0296) (width 1.27) (layer "B.Cu") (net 4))
 (segment (start 152.9461 91.0336) (end 150.3361 91.0336) (width 1.27) (layer "B.Cu") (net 4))
 (segment (start 152.9461 77.0636) (end 152.9461 91.0336) (width 1.27) (layer "B.Cu") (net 4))
 (segment (start 141.5161 114.7036) (end 138.9761 114.7036) (width 1.27) (layer "B.Cu") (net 10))
 (segment (start 128.8161 126.5936) (end 128.8161 141.4526) (width 1.27) (layer "B.Cu") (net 10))
 (segment (start 160.5661 141.4526) (end 159.2961 111.3536) (width 1.27) (layer "B.Cu") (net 10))
 (segment (start 128.8161 141.4526) (end 160.5661 141.4526) (width 1.27) (layer "B.Cu") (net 10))
 (segment (start 138.9761 114.7036) (end 128.8161 126.5936) (width 1.27) (layer "B.Cu") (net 10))
 (segment (start 159.2961 111.3536) (end 150.3361 111.3536) (width 1.27) (layer "B.Cu") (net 10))
 (segment (start 141.5161 118.7036) (end 144.0561 118.9736) (width 1.27) (layer "F.Cu") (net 11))
 (segment (start 145.3261 111.3536) (end 147.7961 111.3536) (width 1.27) (layer "F.Cu") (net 11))
 (segment (start 144.0561 118.9736) (end 145.3261 111.3536) (width 1.27) (layer "F.Cu") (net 11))
 (segment (start 140.2461 109.2736) (end 147.7961 108.8136) (width 1.27) (layer "F.Cu") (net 7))
 (segment (start 140.2461 105.2736) (end 147.7961 103.7336) (width 1.27) (layer "F.Cu") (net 8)))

